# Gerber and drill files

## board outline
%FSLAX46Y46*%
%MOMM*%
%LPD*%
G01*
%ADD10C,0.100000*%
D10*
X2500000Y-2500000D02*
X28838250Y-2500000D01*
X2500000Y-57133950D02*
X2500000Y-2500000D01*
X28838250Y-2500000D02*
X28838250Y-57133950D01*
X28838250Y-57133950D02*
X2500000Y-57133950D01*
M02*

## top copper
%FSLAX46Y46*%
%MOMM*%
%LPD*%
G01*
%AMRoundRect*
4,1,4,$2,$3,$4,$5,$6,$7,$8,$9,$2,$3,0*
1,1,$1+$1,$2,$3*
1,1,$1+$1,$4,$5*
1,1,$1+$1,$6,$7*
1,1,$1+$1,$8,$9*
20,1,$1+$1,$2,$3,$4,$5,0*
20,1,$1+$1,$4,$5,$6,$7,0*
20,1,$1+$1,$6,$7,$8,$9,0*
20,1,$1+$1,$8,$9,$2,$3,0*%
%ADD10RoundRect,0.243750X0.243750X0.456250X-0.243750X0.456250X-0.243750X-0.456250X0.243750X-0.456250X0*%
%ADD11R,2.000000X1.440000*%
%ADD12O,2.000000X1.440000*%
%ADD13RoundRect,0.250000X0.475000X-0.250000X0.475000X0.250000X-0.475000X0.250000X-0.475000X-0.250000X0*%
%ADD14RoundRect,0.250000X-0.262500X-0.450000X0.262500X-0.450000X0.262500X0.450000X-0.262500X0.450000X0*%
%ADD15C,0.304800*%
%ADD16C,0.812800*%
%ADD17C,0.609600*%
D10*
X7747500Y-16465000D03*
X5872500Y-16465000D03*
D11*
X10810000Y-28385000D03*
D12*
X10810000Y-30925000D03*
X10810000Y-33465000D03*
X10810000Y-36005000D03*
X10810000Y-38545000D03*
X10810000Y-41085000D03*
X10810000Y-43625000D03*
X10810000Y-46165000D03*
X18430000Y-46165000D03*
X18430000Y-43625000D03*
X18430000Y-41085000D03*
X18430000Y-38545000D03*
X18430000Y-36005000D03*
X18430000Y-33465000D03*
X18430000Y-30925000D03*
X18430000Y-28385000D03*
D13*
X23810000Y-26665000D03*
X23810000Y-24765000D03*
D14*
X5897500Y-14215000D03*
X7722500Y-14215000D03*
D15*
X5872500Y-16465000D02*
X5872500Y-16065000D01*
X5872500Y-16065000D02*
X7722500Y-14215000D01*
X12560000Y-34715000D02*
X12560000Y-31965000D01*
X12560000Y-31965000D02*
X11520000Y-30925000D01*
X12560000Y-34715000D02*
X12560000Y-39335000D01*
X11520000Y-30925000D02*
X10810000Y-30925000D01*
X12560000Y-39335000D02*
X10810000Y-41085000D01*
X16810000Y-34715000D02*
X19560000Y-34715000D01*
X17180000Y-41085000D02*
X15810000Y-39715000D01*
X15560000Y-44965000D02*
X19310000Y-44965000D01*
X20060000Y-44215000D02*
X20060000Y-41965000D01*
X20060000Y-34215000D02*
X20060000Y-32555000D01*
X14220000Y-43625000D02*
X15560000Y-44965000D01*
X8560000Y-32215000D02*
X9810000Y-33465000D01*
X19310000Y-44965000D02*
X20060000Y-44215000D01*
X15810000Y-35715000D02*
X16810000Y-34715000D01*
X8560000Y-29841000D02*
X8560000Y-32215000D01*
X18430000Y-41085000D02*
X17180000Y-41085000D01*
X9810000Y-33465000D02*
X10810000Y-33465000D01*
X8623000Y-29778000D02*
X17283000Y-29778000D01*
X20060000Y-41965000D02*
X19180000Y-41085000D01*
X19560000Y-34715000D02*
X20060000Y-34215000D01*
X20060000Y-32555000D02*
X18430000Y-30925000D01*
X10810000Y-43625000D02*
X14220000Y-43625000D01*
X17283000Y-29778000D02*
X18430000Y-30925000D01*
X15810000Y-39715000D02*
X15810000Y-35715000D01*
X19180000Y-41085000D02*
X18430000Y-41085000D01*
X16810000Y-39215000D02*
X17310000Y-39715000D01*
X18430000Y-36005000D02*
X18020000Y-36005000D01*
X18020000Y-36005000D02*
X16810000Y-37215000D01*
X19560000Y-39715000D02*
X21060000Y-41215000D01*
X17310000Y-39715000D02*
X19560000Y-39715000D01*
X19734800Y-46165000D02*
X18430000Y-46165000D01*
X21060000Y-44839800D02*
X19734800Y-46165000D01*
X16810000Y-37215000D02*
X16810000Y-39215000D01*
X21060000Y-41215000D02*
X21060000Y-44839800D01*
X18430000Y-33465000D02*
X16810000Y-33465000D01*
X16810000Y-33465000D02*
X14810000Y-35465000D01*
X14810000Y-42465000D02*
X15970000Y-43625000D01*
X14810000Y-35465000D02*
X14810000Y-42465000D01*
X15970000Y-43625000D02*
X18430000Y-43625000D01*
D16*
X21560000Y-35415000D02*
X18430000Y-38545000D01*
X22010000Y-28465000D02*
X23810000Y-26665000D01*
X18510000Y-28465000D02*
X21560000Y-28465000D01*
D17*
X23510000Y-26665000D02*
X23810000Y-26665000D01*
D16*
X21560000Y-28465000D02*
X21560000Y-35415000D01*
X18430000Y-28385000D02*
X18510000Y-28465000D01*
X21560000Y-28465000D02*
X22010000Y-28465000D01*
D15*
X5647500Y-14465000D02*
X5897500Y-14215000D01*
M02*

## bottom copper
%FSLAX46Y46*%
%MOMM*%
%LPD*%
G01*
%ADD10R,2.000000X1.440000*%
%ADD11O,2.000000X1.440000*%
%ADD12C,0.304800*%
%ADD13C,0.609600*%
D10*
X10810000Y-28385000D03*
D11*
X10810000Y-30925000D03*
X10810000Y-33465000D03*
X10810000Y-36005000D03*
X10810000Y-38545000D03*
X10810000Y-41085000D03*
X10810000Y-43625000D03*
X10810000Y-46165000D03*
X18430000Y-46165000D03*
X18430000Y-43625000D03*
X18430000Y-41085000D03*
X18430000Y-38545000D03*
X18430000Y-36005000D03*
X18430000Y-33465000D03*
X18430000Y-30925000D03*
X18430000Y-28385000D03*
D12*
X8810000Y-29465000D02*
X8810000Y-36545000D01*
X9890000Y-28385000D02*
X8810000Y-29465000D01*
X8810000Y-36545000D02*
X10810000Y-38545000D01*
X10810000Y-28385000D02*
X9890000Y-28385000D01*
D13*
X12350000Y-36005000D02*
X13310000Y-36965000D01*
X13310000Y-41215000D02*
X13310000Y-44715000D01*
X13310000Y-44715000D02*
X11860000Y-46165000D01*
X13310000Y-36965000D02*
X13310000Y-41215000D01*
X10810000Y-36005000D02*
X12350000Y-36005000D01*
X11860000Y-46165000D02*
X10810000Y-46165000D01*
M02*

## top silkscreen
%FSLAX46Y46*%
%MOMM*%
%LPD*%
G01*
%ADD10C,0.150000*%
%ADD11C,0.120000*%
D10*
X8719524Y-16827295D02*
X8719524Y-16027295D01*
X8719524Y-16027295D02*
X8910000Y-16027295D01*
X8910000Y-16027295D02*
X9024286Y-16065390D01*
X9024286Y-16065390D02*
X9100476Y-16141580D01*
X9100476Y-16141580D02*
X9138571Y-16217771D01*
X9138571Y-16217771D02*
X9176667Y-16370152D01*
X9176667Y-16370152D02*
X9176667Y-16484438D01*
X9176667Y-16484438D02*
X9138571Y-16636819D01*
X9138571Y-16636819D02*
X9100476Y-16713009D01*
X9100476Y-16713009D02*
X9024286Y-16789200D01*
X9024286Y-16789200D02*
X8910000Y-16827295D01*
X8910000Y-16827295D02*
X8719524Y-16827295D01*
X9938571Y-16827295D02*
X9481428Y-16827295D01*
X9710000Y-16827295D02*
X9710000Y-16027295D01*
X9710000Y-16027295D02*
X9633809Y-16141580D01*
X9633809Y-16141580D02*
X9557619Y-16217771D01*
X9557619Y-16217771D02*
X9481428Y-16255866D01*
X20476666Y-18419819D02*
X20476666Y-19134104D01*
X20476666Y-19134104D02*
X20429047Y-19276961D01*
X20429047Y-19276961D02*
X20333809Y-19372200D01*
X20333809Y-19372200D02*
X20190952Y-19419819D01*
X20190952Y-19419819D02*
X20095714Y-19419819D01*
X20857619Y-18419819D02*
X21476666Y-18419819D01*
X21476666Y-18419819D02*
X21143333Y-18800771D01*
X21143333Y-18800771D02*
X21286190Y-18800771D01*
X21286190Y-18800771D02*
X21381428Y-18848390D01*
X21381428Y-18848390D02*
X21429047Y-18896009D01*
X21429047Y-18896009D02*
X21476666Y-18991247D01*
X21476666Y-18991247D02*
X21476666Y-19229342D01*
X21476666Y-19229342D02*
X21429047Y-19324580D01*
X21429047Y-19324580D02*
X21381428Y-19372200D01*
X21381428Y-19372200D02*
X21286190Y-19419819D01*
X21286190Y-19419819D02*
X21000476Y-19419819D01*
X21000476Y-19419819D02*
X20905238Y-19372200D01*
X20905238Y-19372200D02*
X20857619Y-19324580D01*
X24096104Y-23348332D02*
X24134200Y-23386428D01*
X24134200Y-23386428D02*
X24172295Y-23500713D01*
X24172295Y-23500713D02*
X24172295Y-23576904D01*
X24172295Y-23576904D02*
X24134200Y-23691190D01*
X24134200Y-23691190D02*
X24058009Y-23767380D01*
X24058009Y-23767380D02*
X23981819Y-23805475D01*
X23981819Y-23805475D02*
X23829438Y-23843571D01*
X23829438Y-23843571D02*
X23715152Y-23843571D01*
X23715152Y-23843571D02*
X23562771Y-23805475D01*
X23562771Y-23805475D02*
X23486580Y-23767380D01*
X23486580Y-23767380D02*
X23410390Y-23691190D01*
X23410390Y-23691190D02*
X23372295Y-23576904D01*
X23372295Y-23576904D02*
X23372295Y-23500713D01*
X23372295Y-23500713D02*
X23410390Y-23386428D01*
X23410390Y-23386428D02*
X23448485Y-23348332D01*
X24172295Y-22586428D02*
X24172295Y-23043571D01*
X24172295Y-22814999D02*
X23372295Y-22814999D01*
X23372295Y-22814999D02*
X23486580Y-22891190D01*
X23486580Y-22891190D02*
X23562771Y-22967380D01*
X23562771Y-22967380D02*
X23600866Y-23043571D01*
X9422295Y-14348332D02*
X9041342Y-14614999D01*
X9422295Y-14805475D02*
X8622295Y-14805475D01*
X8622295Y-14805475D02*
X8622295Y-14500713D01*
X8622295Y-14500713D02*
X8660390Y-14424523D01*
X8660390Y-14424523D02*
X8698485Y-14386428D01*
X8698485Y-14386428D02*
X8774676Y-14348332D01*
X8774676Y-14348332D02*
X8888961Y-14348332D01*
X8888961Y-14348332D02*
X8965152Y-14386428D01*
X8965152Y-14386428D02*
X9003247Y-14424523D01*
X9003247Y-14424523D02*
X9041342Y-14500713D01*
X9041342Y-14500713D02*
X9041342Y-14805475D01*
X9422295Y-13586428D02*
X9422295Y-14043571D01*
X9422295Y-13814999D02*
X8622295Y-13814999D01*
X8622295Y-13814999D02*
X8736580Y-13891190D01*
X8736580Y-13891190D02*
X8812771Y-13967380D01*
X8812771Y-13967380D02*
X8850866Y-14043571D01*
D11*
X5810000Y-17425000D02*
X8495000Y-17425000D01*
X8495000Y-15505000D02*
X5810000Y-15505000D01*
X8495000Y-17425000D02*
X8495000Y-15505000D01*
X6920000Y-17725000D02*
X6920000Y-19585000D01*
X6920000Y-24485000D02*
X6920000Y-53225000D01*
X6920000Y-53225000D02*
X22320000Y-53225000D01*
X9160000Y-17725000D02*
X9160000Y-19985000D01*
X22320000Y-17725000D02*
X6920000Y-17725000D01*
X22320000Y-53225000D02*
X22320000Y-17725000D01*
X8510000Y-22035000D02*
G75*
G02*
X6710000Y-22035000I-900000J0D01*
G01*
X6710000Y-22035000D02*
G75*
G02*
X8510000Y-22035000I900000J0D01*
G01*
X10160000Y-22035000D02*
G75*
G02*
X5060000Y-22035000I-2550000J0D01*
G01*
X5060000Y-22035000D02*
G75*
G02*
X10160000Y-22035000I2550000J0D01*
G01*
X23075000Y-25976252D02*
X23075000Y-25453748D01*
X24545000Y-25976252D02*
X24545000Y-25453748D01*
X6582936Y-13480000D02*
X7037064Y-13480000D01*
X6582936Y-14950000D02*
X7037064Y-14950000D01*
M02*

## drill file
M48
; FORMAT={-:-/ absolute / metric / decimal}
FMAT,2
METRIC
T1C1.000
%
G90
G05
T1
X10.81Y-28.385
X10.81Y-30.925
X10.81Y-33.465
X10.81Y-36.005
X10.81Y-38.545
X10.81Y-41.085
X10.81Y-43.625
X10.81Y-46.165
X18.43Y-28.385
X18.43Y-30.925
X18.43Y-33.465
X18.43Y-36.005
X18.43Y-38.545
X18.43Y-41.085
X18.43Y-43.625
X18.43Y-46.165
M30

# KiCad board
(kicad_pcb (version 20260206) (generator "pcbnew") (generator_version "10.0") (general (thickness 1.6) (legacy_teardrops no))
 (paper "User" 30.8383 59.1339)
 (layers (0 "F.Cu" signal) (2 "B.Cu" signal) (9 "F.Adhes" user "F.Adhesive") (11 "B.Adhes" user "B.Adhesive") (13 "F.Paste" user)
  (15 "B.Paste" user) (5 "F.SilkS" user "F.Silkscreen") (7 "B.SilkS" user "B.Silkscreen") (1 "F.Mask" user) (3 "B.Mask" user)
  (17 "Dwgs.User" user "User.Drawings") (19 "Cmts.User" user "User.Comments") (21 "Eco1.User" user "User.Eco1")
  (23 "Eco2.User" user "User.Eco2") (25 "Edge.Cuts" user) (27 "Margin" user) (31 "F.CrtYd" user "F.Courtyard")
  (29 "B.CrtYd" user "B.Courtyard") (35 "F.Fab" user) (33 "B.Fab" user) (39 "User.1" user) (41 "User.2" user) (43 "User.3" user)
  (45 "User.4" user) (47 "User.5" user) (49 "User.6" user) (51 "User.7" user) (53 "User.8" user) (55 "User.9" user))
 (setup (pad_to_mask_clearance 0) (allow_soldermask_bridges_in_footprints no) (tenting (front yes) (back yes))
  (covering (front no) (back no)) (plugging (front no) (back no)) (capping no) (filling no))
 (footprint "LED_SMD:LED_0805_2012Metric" (layer "F.Cu") (at 6.81 16.465 180)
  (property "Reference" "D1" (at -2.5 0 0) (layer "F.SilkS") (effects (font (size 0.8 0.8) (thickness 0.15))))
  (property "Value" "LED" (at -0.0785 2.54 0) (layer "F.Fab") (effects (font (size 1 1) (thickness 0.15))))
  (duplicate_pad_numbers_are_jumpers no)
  (fp_line (start 1 -0.96) (end -1.685 -0.96) (stroke (width 0.12) (type solid)) (layer "F.SilkS"))
  (fp_line (start -1.685 0.96) (end 1 0.96) (stroke (width 0.12) (type solid)) (layer "F.SilkS"))
  (fp_line (start -1.685 -0.96) (end -1.685 0.96) (stroke (width 0.12) (type solid)) (layer "F.SilkS"))
  (pad "1" smd roundrect (at -0.9375 0 180) (size 0.975 1.4) (layers "F.Cu" "F.Mask" "F.Paste") (roundrect_rratio 0.25) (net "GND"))
  (pad "2" smd roundrect (at 0.9375 0 180) (size 0.975 1.4) (layers "F.Cu" "F.Mask" "F.Paste") (roundrect_rratio 0.25) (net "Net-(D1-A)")))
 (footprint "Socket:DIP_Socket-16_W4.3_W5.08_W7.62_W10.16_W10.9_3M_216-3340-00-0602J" (layer "F.Cu") (at 10.81 28.385)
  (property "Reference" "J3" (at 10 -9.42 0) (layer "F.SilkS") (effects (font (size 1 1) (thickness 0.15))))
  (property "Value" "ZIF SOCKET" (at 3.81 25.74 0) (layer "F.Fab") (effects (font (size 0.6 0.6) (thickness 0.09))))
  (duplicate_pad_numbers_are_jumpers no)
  (fp_line (start -3.89 -10.66) (end -3.89 -8.8) (stroke (width 0.12) (type solid)) (layer "F.SilkS"))
  (fp_line (start -3.89 -3.9) (end -3.89 24.84) (stroke (width 0.12) (type solid)) (layer "F.SilkS"))
  (fp_line (start -3.89 24.84) (end 11.51 24.84) (stroke (width 0.12) (type solid)) (layer "F.SilkS"))
  (fp_line (start -1.65 -10.66) (end -1.65 -8.4) (stroke (width 0.12) (type solid)) (layer "F.SilkS"))
  (fp_line (start 11.51 -10.66) (end -3.89 -10.66) (stroke (width 0.12) (type solid)) (layer "F.SilkS"))
  (fp_line (start 11.51 24.84) (end 11.51 -10.66) (stroke (width 0.12) (type solid)) (layer "F.SilkS"))
  (fp_circle (center -3.2 -6.35) (end -2.3 -6.35) (stroke (width 0.12) (type solid)) (fill no) (layer "F.SilkS"))
  (fp_circle (center -3.2 -6.35) (end -0.65 -6.35) (stroke (width 0.12) (type solid)) (fill no) (layer "F.SilkS"))
  (pad "1" thru_hole rect (at 0 0) (size 2 1.44) (drill 1) (layers "*.Cu" "*.Mask") (remove_unused_layers no) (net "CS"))
  (pad "2" thru_hole oval (at 0 2.54) (size 2 1.44) (drill 1) (layers "*.Cu" "*.Mask") (remove_unused_layers no) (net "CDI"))
  (pad "3" thru_hole oval (at 0 5.08) (size 2 1.44) (drill 1) (layers "*.Cu" "*.Mask") (remove_unused_layers no) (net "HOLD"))
  (pad "4" thru_hole oval (at 0 7.62) (size 2 1.44) (drill 1) (layers "*.Cu" "*.Mask") (remove_unused_layers no) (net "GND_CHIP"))
  (pad "5" thru_hole oval (at 0 10.16) (size 2 1.44) (drill 1) (layers "*.Cu" "*.Mask") (remove_unused_layers no) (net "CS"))
  (pad "6" thru_hole oval (at 0 12.7) (size 2 1.44) (drill 1) (layers "*.Cu" "*.Mask") (remove_unused_layers no) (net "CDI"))
  (pad "7" thru_hole oval (at 0 15.24) (size 2 1.44) (drill 1) (layers "*.Cu" "*.Mask") (remove_unused_layers no) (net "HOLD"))
  (pad "8" thru_hole oval (at 0 17.78) (size 2 1.44) (drill 1) (layers "*.Cu" "*.Mask") (remove_unused_layers no) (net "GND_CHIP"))
  (pad "9" thru_hole oval (at 7.62 17.78) (size 2 1.44) (drill 1) (layers "*.Cu" "*.Mask") (remove_unused_layers no) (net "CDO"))
  (pad "10" thru_hole oval (at 7.62 15.24) (size 2 1.44) (drill 1) (layers "*.Cu" "*.Mask") (remove_unused_layers no) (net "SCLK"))
  (pad "11" thru_hole oval (at 7.62 12.7) (size 2 1.44) (drill 1) (layers "*.Cu" "*.Mask") (remove_unused_layers no) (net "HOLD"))
  (pad "12" thru_hole oval (at 7.62 10.16) (size 2 1.44) (drill 1) (layers "*.Cu" "*.Mask") (remove_unused_layers no) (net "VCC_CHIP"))
  (pad "13" thru_hole oval (at 7.62 7.62) (size 2 1.44) (drill 1) (layers "*.Cu" "*.Mask") (remove_unused_layers no) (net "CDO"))
  (pad "14" thru_hole oval (at 7.62 5.08) (size 2 1.44) (drill 1) (layers "*.Cu" "*.Mask") (remove_unused_layers no) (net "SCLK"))
  (pad "15" thru_hole oval (at 7.62 2.54) (size 2 1.44) (drill 1) (layers "*.Cu" "*.Mask") (remove_unused_layers no) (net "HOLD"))
  (pad "16" thru_hole oval (at 7.62 0) (size 2 1.44) (drill 1) (layers "*.Cu" "*.Mask") (remove_unused_layers no) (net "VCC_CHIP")))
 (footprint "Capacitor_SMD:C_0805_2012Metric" (layer "F.Cu") (at 23.81 25.715 90)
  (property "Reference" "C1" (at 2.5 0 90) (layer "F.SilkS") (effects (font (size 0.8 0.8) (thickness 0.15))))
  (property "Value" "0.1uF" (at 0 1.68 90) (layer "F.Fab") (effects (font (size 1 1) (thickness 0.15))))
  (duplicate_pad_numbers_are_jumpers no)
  (fp_line (start -0.261252 -0.735) (end 0.261252 -0.735) (stroke (width 0.12) (type solid)) (layer "F.SilkS"))
  (fp_line (start -0.261252 0.735) (end 0.261252 0.735) (stroke (width 0.12) (type solid)) (layer "F.SilkS"))
  (pad "1" smd roundrect (at -0.95 0 90) (size 1 1.45) (layers "F.Cu" "F.Mask" "F.Paste") (roundrect_rratio 0.25) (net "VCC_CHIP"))
  (pad "2" smd roundrect (at 0.95 0 90) (size 1 1.45) (layers "F.Cu" "F.Mask" "F.Paste") (roundrect_rratio 0.25) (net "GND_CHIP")))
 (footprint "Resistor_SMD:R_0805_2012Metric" (layer "F.Cu") (at 6.81 14.215)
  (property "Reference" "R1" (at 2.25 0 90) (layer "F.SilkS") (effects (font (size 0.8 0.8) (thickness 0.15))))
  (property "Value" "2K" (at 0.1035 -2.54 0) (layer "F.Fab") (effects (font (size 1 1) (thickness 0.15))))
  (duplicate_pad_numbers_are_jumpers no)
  (fp_line (start -0.227064 -0.735) (end 0.227064 -0.735) (stroke (width 0.12) (type solid)) (layer "F.SilkS"))
  (fp_line (start -0.227064 0.735) (end 0.227064 0.735) (stroke (width 0.12) (type solid)) (layer "F.SilkS"))
  (pad "1" smd roundrect (at -0.9125 0) (size 1.025 1.4) (layers "F.Cu" "F.Mask" "F.Paste") (roundrect_rratio 0.243902439) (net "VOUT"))
  (pad "2" smd roundrect (at 0.9125 0) (size 1.025 1.4) (layers "F.Cu" "F.Mask" "F.Paste") (roundrect_rratio 0.243902439) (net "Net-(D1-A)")))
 (gr_line (start 2.5 2.5) (end 28.83825 2.5) (stroke (width 0.1) (type default)) (layer "Edge.Cuts"))
 (gr_line (start 2.5 57.13395) (end 2.5 2.5) (stroke (width 0.1) (type default)) (layer "Edge.Cuts"))
 (gr_line (start 28.83825 2.5) (end 28.83825 57.13395) (stroke (width 0.1) (type default)) (layer "Edge.Cuts"))
 (gr_line (start 28.83825 57.13395) (end 2.5 57.13395) (stroke (width 0.1) (type default)) (layer "Edge.Cuts"))
 (segment (start 5.8725 16.465) (end 5.8725 16.065) (width 0.3048) (layer "F.Cu") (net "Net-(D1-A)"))
 (segment (start 5.8725 16.065) (end 7.7225 14.215) (width 0.3048) (layer "F.Cu") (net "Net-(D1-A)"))
 (segment (start 8.81 29.465) (end 8.81 36.545) (width 0.3048) (layer "B.Cu") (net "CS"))
 (segment (start 9.89 28.385) (end 8.81 29.465) (width 0.3048) (layer "B.Cu") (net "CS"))
 (segment (start 8.81 36.545) (end 10.81 38.545) (width 0.3048) (layer "B.Cu") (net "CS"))
 (segment (start 10.81 28.385) (end 9.89 28.385) (width 0.3048) (layer "B.Cu") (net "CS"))
 (segment (start 12.56 34.715) (end 12.56 31.965) (width 0.3048) (layer "F.Cu") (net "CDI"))
 (segment (start 12.56 31.965) (end 11.52 30.925) (width 0.3048) (layer "F.Cu") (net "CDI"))
 (segment (start 12.56 34.715) (end 12.56 39.335) (width 0.3048) (layer "F.Cu") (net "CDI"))
 (segment (start 11.52 30.925) (end 10.81 30.925) (width 0.3048) (layer "F.Cu") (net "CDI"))
 (segment (start 12.56 39.335) (end 10.81 41.085) (width 0.3048) (layer "F.Cu") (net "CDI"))
 (segment (start 16.81 34.715) (end 19.56 34.715) (width 0.3048) (layer "F.Cu") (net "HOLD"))
 (segment (start 17.18 41.085) (end 15.81 39.715) (width 0.3048) (layer "F.Cu") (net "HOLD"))
 (segment (start 15.56 44.965) (end 19.31 44.965) (width 0.3048) (layer "F.Cu") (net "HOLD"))
 (segment (start 20.06 44.215) (end 20.06 41.965) (width 0.3048) (layer "F.Cu") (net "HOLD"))
 (segment (start 20.06 34.215) (end 20.06 32.555) (width 0.3048) (layer "F.Cu") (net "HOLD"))
 (segment (start 14.22 43.625) (end 15.56 44.965) (width 0.3048) (layer "F.Cu") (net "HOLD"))
 (segment (start 8.56 32.215) (end 9.81 33.465) (width 0.3048) (layer "F.Cu") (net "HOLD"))
 (segment (start 19.31 44.965) (end 20.06 44.215) (width 0.3048) (layer "F.Cu") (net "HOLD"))
 (segment (start 15.81 35.715) (end 16.81 34.715) (width 0.3048) (layer "F.Cu") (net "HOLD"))
 (segment (start 8.56 29.841) (end 8.56 32.215) (width 0.3048) (layer "F.Cu") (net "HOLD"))
 (segment (start 18.43 41.085) (end 17.18 41.085) (width 0.3048) (layer "F.Cu") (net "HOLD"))
 (segment (start 9.81 33.465) (end 10.81 33.465) (width 0.3048) (layer "F.Cu") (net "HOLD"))
 (segment (start 8.623 29.778) (end 17.283 29.778) (width 0.3048) (layer "F.Cu") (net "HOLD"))
 (segment (start 20.06 41.965) (end 19.18 41.085) (width 0.3048) (layer "F.Cu") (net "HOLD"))
 (segment (start 19.56 34.715) (end 20.06 34.215) (width 0.3048) (layer "F.Cu") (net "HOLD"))
 (segment (start 20.06 32.555) (end 18.43 30.925) (width 0.3048) (layer "F.Cu") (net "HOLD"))
 (segment (start 10.81 43.625) (end 14.22 43.625) (width 0.3048) (layer "F.Cu") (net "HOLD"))
 (segment (start 17.283 29.778) (end 18.43 30.925) (width 0.3048) (layer "F.Cu") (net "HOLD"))
 (segment (start 15.81 39.715) (end 15.81 35.715) (width 0.3048) (layer "F.Cu") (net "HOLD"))
 (segment (start 19.18 41.085) (end 18.43 41.085) (width 0.3048) (layer "F.Cu") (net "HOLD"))
 (segment (start 12.35 36.005) (end 13.31 36.965) (width 0.6096) (layer "B.Cu") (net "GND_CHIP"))
 (segment (start 13.31 41.215) (end 13.31 44.715) (width 0.6096) (layer "B.Cu") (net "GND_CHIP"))
 (segment (start 13.31 44.715) (end 11.86 46.165) (width 0.6096) (layer "B.Cu") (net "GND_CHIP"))
 (segment (start 13.31 36.965) (end 13.31 41.215) (width 0.6096) (layer "B.Cu") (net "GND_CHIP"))
 (segment (start 10.81 36.005) (end 12.35 36.005) (width 0.6096) (layer "B.Cu") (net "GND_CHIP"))
 (segment (start 11.86 46.165) (end 10.81 46.165) (width 0.6096) (layer "B.Cu") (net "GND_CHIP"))
 (segment (start 16.81 39.215) (end 17.31 39.715) (width 0.3048) (layer "F.Cu") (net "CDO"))
 (segment (start 18.43 36.005) (end 18.02 36.005) (width 0.3048) (layer "F.Cu") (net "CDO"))
 (segment (start 18.02 36.005) (end 16.81 37.215) (width 0.3048) (layer "F.Cu") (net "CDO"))
 (segment (start 19.56 39.715) (end 21.06 41.215) (width 0.3048) (layer "F.Cu") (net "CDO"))
 (segment (start 17.31 39.715) (end 19.56 39.715) (width 0.3048) (layer "F.Cu") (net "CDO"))
 (segment (start 19.7348 46.165) (end 18.43 46.165) (width 0.3048) (layer "F.Cu") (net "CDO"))
 (segment (start 21.06 44.8398) (end 19.7348 46.165) (width 0.3048) (layer "F.Cu") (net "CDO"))
 (segment (start 16.81 37.215) (end 16.81 39.215) (width 0.3048) (layer "F.Cu") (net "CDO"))
 (segment (start 21.06 41.215) (end 21.06 44.8398) (width 0.3048) (layer "F.Cu") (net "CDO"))
 (segment (start 18.43 33.465) (end 16.81 33.465) (width 0.3048) (layer "F.Cu") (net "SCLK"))
 (segment (start 16.81 33.465) (end 14.81 35.465) (width 0.3048) (layer "F.Cu") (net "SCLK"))
 (segment (start 14.81 42.465) (end 15.97 43.625) (width 0.3048) (layer "F.Cu") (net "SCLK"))
 (segment (start 14.81 35.465) (end 14.81 42.465) (width 0.3048) (layer "F.Cu") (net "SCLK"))
 (segment (start 15.97 43.625) (end 18.43 43.625) (width 0.3048) (layer "F.Cu") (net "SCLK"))
 (segment (start 21.56 35.415) (end 18.43 38.545) (width 0.8128) (layer "F.Cu") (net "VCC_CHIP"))
 (segment (start 22.01 28.465) (end 23.81 26.665) (width 0.8128) (layer "F.Cu") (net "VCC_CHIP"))
 (segment (start 18.51 28.465) (end 21.56 28.465) (width 0.8128) (layer "F.Cu") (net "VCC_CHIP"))
 (segment (start 23.51 26.665) (end 23.81 26.665) (width 0.6096) (layer "F.Cu") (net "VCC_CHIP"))
 (segment (start 21.56 28.465) (end 21.56 35.415) (width 0.8128) (layer "F.Cu") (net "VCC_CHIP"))
 (segment (start 18.43 28.385) (end 18.51 28.465) (width 0.8128) (layer "F.Cu") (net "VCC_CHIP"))
 (segment (start 21.56 28.465) (end 22.01 28.465) (width 0.8128) (layer "F.Cu") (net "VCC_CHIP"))
 (segment (start 5.6475 14.465) (end 5.8975 14.215) (width 0.3048) (layer "F.Cu") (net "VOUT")))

